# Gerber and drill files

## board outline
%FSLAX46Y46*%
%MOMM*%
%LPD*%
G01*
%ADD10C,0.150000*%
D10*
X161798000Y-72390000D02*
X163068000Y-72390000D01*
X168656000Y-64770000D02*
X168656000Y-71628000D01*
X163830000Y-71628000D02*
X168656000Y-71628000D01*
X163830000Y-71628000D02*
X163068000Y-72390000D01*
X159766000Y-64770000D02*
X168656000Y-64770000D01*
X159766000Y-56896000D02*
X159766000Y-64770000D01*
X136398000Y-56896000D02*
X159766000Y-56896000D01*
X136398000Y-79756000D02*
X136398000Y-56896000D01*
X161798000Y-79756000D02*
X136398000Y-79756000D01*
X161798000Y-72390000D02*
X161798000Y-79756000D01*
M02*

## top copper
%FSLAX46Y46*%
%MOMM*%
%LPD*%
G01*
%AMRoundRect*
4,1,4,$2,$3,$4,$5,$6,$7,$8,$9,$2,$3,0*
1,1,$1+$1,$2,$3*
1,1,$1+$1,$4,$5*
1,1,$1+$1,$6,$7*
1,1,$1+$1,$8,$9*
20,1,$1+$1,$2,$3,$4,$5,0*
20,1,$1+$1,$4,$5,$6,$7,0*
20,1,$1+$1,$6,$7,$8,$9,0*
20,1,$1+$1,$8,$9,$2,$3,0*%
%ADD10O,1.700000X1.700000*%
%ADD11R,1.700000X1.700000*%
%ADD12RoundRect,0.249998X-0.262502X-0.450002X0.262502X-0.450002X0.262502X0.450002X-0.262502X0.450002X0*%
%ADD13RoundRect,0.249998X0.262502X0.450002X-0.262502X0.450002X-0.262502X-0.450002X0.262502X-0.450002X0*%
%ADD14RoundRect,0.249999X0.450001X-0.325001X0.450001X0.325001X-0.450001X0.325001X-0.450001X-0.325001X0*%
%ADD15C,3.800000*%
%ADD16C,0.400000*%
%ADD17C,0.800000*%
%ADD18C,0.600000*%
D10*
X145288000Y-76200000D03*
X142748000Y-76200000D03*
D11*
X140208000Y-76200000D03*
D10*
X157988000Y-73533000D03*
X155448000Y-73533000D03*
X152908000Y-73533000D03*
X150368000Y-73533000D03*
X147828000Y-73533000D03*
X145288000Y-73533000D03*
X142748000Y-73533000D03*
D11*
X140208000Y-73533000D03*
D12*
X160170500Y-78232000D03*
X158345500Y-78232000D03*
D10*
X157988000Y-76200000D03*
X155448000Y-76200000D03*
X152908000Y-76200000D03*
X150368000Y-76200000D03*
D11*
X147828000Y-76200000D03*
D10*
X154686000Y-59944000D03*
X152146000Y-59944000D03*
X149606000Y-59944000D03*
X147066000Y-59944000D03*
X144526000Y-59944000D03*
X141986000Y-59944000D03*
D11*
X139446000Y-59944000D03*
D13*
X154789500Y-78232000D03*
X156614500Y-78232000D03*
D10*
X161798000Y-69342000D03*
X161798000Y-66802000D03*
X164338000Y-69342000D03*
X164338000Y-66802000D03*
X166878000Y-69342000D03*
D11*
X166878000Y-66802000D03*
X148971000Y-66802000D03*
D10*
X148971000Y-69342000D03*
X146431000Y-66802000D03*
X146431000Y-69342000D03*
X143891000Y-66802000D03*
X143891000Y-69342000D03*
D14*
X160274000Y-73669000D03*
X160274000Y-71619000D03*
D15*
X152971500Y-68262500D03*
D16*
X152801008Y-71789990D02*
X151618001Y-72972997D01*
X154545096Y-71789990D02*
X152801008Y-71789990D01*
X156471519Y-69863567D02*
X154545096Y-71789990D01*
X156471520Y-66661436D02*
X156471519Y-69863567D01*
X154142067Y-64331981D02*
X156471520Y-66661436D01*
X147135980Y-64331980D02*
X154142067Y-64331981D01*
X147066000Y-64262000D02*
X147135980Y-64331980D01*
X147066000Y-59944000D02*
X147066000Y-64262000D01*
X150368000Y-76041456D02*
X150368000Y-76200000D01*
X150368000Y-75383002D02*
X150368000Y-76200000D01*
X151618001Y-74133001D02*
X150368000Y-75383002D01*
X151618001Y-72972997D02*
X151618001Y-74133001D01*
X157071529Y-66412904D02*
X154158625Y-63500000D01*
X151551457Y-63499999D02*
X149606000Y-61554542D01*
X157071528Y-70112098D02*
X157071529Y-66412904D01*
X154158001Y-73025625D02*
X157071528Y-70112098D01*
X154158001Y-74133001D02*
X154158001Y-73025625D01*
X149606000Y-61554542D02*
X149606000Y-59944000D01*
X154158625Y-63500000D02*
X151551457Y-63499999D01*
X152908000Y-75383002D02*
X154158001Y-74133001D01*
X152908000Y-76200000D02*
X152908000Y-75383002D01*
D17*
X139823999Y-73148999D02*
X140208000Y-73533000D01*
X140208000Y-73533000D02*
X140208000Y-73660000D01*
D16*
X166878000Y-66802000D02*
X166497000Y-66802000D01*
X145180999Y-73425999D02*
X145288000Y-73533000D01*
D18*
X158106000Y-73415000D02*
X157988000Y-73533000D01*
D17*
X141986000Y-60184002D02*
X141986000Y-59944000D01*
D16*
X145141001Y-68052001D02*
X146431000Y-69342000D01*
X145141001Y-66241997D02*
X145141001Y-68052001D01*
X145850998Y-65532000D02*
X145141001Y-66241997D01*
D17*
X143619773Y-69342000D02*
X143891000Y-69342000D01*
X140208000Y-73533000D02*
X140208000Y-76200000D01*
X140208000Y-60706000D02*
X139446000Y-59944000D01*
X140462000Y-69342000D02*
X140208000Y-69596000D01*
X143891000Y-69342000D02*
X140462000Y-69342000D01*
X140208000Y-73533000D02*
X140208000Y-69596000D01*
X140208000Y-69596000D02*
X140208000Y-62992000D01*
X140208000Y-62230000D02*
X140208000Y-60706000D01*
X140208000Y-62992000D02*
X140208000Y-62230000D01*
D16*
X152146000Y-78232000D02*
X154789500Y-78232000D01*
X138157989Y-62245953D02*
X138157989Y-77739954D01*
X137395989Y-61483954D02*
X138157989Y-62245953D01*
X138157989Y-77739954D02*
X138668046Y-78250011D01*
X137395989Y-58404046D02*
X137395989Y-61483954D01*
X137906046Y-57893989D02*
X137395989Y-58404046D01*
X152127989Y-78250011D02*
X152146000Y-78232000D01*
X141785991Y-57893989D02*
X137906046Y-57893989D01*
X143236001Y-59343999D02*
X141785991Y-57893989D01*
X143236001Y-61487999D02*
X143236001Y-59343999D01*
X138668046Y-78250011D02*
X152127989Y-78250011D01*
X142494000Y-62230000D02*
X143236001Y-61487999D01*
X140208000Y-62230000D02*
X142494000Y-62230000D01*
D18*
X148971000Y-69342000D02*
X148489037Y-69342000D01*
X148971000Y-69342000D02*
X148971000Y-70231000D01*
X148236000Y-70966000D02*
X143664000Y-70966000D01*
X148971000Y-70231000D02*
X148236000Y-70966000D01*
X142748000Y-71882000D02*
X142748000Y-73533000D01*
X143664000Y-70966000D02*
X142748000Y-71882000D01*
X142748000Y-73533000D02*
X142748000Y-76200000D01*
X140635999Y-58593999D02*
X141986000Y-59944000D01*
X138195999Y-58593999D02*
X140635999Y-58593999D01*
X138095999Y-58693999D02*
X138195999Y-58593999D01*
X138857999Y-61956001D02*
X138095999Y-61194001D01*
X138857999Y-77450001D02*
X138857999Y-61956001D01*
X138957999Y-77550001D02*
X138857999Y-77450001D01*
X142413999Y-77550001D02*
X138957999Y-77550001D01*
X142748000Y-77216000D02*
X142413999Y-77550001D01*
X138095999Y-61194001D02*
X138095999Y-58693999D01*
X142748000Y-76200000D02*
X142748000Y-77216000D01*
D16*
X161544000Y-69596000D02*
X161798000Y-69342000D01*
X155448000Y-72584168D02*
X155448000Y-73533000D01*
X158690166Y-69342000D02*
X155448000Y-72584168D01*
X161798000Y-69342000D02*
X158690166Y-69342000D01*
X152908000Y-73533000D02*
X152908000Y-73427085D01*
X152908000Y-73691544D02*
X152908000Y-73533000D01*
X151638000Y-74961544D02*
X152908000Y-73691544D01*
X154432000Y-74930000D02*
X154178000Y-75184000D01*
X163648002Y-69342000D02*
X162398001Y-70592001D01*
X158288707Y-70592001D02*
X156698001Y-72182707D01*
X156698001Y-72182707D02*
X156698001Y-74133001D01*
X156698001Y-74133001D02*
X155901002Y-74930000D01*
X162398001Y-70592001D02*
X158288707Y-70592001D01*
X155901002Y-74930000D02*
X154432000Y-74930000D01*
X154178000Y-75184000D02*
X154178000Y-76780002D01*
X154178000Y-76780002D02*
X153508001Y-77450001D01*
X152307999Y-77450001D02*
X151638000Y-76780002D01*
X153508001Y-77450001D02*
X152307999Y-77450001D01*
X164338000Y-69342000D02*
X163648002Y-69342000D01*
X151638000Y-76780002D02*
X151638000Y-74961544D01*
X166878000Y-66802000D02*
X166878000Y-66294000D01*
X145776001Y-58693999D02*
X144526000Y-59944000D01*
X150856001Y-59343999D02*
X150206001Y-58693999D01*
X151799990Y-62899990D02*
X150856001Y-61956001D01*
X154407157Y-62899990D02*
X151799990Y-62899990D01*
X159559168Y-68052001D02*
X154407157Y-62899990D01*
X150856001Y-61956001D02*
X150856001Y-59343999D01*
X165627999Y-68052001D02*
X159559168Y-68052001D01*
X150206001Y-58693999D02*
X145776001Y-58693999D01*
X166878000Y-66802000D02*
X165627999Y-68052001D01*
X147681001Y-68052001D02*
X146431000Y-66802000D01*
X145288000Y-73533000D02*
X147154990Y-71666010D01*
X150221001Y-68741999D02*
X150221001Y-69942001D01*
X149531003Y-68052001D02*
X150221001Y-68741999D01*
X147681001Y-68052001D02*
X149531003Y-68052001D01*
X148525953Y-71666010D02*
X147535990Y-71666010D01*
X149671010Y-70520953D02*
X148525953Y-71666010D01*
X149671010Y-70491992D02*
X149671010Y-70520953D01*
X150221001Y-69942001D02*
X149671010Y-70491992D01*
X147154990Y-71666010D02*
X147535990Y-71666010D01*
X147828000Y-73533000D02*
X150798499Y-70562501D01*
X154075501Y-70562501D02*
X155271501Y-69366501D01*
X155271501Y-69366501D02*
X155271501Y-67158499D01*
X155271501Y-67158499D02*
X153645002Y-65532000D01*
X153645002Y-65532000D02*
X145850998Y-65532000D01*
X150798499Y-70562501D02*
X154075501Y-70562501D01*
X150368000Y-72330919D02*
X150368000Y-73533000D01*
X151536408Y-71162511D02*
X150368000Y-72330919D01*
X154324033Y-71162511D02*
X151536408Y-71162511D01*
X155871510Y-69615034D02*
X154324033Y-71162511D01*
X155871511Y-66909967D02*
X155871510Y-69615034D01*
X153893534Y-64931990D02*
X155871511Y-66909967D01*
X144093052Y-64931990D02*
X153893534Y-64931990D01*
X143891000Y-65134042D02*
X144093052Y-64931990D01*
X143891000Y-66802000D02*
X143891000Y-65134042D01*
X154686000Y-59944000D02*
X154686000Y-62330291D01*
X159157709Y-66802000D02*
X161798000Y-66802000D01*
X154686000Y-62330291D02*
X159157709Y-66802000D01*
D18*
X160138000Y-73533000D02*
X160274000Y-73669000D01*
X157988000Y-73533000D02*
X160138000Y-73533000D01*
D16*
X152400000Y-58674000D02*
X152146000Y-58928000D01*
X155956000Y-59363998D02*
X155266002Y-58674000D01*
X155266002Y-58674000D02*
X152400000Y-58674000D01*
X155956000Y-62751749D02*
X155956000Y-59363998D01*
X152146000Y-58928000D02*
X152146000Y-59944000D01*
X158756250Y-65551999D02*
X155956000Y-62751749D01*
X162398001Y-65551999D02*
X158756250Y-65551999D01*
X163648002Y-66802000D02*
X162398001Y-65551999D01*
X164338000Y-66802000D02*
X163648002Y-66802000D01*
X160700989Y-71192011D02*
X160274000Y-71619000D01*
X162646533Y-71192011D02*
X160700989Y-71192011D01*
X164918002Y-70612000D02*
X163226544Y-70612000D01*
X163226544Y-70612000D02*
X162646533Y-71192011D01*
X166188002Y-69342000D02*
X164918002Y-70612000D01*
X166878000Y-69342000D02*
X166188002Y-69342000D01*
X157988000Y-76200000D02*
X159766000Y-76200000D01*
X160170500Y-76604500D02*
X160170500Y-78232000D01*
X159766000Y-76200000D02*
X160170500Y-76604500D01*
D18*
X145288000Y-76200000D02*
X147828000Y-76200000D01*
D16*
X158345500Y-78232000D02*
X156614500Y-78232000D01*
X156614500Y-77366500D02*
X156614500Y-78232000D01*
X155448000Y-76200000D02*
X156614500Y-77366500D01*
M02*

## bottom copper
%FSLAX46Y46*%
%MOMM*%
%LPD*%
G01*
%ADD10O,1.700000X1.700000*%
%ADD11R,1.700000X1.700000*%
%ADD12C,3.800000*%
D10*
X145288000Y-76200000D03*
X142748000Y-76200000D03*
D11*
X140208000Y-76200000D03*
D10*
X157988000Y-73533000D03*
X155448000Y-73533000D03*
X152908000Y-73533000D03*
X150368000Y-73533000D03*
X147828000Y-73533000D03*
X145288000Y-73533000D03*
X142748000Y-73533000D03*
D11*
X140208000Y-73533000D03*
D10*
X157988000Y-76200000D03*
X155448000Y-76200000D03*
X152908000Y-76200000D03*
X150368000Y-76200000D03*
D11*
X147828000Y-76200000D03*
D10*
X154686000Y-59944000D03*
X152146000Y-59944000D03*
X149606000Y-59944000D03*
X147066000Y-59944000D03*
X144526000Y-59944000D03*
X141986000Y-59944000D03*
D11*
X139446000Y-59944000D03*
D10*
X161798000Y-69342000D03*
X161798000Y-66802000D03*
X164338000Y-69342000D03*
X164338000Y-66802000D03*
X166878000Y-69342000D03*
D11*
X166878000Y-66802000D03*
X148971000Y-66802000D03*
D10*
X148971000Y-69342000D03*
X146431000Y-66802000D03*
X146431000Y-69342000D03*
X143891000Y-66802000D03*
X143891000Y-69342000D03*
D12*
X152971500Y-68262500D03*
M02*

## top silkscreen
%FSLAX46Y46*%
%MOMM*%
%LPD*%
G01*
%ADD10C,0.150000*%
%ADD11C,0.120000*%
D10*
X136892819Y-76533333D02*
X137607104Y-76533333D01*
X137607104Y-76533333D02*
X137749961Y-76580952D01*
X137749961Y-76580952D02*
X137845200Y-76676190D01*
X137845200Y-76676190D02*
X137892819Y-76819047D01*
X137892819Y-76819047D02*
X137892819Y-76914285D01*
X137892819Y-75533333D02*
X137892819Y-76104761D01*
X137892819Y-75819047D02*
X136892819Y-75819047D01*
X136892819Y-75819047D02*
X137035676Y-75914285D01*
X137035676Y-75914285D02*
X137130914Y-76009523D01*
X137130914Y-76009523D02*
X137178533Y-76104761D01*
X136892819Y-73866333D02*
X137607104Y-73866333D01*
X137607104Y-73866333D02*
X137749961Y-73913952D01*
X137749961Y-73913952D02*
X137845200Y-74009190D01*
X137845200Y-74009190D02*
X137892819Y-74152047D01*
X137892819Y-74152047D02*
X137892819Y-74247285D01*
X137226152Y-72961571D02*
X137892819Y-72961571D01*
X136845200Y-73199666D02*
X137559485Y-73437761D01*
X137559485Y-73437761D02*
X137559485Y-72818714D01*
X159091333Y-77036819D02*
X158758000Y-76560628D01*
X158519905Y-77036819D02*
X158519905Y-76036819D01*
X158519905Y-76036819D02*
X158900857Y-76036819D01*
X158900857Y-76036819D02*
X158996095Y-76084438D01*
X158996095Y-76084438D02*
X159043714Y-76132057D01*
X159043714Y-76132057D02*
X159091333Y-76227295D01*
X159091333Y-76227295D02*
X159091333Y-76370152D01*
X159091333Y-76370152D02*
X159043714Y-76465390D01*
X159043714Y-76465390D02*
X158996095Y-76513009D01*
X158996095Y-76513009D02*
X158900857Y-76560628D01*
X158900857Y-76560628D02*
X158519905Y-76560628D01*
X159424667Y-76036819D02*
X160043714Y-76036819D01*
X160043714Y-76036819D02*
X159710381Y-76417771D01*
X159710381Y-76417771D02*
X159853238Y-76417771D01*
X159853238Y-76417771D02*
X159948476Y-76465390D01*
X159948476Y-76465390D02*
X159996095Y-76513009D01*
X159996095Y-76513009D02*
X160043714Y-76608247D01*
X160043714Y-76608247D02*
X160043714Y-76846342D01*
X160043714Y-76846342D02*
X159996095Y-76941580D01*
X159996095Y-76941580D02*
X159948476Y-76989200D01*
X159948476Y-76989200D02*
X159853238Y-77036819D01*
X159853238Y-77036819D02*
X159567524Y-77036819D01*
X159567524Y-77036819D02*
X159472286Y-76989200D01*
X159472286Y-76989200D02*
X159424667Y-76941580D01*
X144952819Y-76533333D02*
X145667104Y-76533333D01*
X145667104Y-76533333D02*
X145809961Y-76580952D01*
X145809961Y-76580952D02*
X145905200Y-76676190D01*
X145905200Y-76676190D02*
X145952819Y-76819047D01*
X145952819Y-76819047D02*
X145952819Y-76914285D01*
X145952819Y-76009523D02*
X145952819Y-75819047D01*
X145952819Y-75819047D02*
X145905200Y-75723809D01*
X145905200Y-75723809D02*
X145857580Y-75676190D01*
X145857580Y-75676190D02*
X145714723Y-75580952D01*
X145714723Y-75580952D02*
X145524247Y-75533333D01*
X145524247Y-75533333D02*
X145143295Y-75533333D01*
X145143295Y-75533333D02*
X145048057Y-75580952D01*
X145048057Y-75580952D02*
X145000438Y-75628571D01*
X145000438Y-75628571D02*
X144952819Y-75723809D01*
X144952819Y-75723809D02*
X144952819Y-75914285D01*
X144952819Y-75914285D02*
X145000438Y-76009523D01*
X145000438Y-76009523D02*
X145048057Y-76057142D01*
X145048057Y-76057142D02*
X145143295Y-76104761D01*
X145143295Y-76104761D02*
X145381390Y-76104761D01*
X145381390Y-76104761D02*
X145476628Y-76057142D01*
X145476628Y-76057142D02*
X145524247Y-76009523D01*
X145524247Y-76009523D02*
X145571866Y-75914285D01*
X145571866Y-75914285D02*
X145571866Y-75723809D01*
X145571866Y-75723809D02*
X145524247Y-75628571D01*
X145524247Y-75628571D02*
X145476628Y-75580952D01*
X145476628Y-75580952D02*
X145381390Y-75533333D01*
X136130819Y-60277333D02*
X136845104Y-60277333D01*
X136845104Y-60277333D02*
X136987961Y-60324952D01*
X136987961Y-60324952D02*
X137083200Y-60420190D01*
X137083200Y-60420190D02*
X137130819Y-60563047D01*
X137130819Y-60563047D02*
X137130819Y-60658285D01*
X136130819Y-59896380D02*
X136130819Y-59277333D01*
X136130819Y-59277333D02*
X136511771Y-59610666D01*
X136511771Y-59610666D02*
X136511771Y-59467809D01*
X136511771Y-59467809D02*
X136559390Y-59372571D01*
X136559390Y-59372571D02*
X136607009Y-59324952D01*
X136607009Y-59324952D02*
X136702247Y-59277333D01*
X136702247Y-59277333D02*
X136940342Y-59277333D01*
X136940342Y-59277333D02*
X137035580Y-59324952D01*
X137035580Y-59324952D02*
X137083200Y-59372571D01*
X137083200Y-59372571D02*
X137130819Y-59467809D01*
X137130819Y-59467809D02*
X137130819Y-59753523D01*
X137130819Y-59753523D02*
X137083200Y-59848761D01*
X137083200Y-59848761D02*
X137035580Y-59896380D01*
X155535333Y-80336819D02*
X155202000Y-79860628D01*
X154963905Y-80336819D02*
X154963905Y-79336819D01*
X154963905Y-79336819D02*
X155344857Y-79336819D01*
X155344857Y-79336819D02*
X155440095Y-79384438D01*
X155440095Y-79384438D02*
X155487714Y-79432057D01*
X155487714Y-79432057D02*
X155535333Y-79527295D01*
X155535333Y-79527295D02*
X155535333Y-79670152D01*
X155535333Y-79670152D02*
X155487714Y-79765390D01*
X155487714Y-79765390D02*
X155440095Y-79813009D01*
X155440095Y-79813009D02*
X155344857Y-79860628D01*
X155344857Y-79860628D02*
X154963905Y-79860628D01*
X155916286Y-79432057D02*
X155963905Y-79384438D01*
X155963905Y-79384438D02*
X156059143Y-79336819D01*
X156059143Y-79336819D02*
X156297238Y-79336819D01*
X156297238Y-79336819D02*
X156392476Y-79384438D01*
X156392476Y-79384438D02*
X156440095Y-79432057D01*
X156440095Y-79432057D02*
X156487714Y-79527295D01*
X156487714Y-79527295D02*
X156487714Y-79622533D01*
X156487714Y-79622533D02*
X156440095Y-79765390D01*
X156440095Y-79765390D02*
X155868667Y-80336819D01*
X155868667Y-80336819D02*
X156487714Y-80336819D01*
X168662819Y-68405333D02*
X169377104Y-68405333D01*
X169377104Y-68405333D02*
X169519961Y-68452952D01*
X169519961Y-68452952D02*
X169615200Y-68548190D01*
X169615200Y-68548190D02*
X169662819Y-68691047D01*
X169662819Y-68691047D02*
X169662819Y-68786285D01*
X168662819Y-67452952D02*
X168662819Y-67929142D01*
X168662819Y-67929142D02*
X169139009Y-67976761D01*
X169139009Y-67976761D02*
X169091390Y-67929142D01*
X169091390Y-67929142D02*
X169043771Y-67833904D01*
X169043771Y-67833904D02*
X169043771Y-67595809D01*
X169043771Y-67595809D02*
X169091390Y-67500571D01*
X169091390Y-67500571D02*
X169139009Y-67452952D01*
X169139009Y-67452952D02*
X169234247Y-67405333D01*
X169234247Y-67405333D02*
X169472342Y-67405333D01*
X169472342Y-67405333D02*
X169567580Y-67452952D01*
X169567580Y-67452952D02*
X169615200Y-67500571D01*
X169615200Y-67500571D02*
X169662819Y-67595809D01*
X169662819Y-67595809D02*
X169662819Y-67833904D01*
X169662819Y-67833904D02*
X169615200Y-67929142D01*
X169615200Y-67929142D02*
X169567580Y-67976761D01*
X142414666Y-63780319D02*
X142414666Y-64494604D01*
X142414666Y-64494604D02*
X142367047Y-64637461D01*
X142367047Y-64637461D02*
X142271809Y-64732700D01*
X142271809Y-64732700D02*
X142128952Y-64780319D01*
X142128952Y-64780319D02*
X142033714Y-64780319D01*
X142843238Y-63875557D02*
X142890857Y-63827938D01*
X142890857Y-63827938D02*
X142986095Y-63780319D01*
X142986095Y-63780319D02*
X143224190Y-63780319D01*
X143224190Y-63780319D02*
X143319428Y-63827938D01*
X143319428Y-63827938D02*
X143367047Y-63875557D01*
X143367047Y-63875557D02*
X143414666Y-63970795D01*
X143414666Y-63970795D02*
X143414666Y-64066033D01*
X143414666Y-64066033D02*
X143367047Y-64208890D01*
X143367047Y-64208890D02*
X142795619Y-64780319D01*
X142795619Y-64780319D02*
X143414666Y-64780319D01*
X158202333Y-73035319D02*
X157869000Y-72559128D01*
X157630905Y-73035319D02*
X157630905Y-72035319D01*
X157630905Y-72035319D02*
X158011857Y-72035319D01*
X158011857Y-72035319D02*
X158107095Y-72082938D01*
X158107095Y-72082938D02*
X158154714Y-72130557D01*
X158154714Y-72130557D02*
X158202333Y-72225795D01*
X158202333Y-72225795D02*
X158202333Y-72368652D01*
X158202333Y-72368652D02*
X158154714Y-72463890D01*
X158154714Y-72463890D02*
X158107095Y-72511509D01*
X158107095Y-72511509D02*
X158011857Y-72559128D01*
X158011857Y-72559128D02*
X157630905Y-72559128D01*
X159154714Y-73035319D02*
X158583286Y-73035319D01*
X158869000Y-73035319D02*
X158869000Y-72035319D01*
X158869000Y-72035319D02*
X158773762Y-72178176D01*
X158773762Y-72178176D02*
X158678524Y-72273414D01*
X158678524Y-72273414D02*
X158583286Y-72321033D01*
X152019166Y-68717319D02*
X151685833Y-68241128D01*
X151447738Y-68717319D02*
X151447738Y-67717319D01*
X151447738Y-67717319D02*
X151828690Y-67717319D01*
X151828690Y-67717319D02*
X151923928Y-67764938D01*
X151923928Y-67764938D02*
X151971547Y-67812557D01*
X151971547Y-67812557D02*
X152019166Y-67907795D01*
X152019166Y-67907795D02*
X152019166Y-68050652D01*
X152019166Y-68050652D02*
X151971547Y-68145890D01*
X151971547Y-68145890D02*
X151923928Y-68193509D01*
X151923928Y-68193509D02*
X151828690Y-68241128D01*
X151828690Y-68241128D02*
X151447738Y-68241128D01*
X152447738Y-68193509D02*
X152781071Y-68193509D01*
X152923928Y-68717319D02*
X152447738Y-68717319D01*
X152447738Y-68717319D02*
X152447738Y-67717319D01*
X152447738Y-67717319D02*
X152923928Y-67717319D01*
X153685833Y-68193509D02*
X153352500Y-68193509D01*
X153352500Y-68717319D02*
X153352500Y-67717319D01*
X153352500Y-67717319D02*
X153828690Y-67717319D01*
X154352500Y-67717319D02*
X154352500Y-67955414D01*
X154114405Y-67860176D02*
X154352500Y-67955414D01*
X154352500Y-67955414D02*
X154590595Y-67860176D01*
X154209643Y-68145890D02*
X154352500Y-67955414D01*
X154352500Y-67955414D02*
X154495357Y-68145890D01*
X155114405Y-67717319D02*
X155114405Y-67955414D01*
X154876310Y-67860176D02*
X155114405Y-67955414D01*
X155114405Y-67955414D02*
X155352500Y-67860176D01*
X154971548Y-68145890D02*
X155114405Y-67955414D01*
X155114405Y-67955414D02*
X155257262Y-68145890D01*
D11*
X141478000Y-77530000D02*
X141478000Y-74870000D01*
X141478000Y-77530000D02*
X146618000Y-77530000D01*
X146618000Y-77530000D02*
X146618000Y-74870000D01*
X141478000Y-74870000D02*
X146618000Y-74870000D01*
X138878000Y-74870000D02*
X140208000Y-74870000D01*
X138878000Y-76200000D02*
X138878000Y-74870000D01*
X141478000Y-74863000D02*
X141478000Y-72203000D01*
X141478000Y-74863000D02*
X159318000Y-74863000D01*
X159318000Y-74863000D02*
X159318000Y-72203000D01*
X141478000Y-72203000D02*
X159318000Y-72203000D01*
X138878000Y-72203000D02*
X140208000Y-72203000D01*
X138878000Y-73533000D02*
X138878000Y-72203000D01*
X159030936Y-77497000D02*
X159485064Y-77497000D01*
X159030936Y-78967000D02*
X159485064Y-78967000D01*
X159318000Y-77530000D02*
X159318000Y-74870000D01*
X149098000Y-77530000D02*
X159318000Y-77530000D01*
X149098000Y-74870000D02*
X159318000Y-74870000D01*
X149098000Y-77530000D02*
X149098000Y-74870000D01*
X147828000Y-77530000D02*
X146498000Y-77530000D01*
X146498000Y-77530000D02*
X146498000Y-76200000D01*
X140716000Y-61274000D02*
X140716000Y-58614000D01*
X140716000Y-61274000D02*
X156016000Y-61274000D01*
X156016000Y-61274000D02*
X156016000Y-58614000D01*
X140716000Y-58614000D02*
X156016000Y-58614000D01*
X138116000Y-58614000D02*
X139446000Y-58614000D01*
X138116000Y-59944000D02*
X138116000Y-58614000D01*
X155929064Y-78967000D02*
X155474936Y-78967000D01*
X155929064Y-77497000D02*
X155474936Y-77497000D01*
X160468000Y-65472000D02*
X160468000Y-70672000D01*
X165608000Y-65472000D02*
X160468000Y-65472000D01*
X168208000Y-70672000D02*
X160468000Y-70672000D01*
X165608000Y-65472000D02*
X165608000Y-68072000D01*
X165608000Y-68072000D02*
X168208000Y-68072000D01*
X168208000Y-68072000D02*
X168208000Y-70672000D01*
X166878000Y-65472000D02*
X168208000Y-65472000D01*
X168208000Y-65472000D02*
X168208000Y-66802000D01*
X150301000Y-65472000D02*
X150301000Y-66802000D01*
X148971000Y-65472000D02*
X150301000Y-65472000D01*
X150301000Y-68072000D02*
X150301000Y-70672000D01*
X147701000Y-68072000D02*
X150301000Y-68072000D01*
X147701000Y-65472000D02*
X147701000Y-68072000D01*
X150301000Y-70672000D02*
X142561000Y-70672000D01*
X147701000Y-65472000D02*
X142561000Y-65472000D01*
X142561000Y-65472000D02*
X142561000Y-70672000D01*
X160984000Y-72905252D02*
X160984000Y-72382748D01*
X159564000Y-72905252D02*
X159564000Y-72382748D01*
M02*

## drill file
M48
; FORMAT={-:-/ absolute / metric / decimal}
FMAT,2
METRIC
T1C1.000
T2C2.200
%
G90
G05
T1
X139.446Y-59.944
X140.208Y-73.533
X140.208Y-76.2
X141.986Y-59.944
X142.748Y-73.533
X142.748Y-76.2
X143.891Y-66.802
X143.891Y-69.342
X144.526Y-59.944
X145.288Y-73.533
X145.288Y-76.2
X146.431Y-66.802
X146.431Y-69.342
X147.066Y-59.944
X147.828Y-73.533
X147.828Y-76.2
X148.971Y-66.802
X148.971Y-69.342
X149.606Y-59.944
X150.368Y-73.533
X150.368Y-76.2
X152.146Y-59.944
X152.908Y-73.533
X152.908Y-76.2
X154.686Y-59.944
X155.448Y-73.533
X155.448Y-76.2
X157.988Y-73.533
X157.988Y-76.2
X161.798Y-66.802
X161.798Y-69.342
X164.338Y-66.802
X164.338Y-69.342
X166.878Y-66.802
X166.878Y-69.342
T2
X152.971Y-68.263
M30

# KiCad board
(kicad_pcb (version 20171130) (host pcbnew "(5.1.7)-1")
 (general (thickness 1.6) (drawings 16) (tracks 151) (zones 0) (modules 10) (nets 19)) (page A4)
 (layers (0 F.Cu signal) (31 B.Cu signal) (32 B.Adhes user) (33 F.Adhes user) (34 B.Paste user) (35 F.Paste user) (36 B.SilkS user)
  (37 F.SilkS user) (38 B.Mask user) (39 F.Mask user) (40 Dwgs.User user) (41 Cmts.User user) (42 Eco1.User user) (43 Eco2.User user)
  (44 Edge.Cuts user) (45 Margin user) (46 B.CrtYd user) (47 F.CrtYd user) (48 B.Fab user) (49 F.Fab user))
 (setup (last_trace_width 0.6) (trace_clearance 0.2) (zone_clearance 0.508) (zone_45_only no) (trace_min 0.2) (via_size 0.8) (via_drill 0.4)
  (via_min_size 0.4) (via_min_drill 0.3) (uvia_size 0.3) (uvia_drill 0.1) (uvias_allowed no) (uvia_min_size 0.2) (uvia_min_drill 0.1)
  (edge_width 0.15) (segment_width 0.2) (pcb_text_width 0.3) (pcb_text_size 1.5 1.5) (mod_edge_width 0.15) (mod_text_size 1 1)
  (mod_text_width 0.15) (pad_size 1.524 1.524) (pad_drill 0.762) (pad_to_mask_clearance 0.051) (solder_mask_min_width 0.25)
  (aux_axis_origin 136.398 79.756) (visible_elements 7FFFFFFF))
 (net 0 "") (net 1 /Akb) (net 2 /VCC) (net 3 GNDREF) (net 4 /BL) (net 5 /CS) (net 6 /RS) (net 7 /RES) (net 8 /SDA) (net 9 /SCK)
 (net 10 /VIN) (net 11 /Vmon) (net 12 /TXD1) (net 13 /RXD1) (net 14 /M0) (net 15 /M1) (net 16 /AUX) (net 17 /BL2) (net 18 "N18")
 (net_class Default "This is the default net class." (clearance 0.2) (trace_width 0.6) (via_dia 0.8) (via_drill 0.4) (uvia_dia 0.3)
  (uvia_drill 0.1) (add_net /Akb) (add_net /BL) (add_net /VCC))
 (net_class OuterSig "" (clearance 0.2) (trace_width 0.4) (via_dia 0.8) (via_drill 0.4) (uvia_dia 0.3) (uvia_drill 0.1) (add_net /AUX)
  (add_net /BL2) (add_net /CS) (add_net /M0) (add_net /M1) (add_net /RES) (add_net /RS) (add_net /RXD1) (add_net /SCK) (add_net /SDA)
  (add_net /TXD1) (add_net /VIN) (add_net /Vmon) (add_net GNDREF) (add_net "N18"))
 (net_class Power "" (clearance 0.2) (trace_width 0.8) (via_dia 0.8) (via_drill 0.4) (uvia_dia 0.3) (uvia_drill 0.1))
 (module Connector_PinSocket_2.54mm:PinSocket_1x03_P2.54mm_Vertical (layer F.Cu) (at 140.208 76.2 90)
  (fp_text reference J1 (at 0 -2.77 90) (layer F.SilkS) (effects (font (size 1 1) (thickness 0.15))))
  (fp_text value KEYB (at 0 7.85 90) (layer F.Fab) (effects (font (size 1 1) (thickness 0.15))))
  (fp_line (start -1.33 1.27) (end 1.33 1.27) (layer F.SilkS) (width 0.12))
  (fp_line (start -1.33 1.27) (end -1.33 6.41) (layer F.SilkS) (width 0.12))
  (fp_line (start -1.33 6.41) (end 1.33 6.41) (layer F.SilkS) (width 0.12))
  (fp_line (start 1.33 1.27) (end 1.33 6.41) (layer F.SilkS) (width 0.12))
  (fp_line (start 1.33 -1.33) (end 1.33 0) (layer F.SilkS) (width 0.12))
  (fp_line (start 0 -1.33) (end 1.33 -1.33) (layer F.SilkS) (width 0.12))
  (pad 3 thru_hole oval (at 0 5.08 90) (size 1.7 1.7) (drill 1) (layers *.Cu *.Mask) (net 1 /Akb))
  (pad 2 thru_hole oval (at 0 2.54 90) (size 1.7 1.7) (drill 1) (layers *.Cu *.Mask) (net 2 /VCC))
  (pad 1 thru_hole rect (at 0 0 90) (size 1.7 1.7) (drill 1) (layers *.Cu *.Mask) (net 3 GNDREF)))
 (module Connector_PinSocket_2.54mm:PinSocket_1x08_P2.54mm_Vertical (layer F.Cu) (at 140.208 73.533 90)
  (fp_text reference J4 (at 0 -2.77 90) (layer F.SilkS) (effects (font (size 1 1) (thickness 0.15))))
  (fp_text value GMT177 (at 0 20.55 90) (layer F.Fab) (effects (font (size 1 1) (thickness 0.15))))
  (fp_line (start -1.33 1.27) (end 1.33 1.27) (layer F.SilkS) (width 0.12))
  (fp_line (start -1.33 1.27) (end -1.33 19.11) (layer F.SilkS) (width 0.12))
  (fp_line (start -1.33 19.11) (end 1.33 19.11) (layer F.SilkS) (width 0.12))
  (fp_line (start 1.33 1.27) (end 1.33 19.11) (layer F.SilkS) (width 0.12))
  (fp_line (start 1.33 -1.33) (end 1.33 0) (layer F.SilkS) (width 0.12))
  (fp_line (start 0 -1.33) (end 1.33 -1.33) (layer F.SilkS) (width 0.12))
  (pad 8 thru_hole oval (at 0 17.78 90) (size 1.7 1.7) (drill 1) (layers *.Cu *.Mask) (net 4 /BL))
  (pad 7 thru_hole oval (at 0 15.24 90) (size 1.7 1.7) (drill 1) (layers *.Cu *.Mask) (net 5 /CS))
  (pad 6 thru_hole oval (at 0 12.7 90) (size 1.7 1.7) (drill 1) (layers *.Cu *.Mask) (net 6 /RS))
  (pad 5 thru_hole oval (at 0 10.16 90) (size 1.7 1.7) (drill 1) (layers *.Cu *.Mask) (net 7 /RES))
  (pad 4 thru_hole oval (at 0 7.62 90) (size 1.7 1.7) (drill 1) (layers *.Cu *.Mask) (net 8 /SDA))
  (pad 3 thru_hole oval (at 0 5.08 90) (size 1.7 1.7) (drill 1) (layers *.Cu *.Mask) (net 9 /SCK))
  (pad 2 thru_hole oval (at 0 2.54 90) (size 1.7 1.7) (drill 1) (layers *.Cu *.Mask) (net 2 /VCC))
  (pad 1 thru_hole rect (at 0 0 90) (size 1.7 1.7) (drill 1) (layers *.Cu *.Mask) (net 3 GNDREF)))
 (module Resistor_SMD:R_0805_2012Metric (layer F.Cu) (at 159.258 78.232)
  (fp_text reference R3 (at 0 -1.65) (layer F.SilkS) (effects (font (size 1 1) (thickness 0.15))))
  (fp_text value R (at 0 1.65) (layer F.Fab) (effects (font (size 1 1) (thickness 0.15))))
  (fp_line (start -0.227064 -0.735) (end 0.227064 -0.735) (layer F.SilkS) (width 0.12))
  (fp_line (start -0.227064 0.735) (end 0.227064 0.735) (layer F.SilkS) (width 0.12))
  (pad 2 smd roundrect (at 0.9125 0) (size 1.025 1.4) (layers F.Cu F.Paste F.Mask) (roundrect_rratio 0.2439004878048781) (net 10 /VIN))
  (pad 1 smd roundrect (at -0.9125 0) (size 1.025 1.4) (layers F.Cu F.Paste F.Mask) (roundrect_rratio 0.2439004878048781) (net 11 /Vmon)))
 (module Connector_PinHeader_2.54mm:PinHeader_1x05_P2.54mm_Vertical (layer F.Cu) (at 147.828 76.2 90)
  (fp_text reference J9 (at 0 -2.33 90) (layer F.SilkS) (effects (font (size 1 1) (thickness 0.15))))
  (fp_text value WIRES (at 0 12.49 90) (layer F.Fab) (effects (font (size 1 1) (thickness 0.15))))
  (fp_line (start -1.33 11.49) (end 1.33 11.49) (layer F.SilkS) (width 0.12))
  (fp_line (start -1.33 1.27) (end -1.33 11.49) (layer F.SilkS) (width 0.12))
  (fp_line (start 1.33 1.27) (end 1.33 11.49) (layer F.SilkS) (width 0.12))
  (fp_line (start -1.33 1.27) (end 1.33 1.27) (layer F.SilkS) (width 0.12))
  (fp_line (start -1.33 0) (end -1.33 -1.33) (layer F.SilkS) (width 0.12))
  (fp_line (start -1.33 -1.33) (end 0 -1.33) (layer F.SilkS) (width 0.12))
  (pad 5 thru_hole oval (at 0 10.16 90) (size 1.7 1.7) (drill 1) (layers *.Cu *.Mask) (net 10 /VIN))
  (pad 4 thru_hole oval (at 0 7.62 90) (size 1.7 1.7) (drill 1) (layers *.Cu *.Mask) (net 11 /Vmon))
  (pad 3 thru_hole oval (at 0 5.08 90) (size 1.7 1.7) (drill 1) (layers *.Cu *.Mask) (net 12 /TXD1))
  (pad 2 thru_hole oval (at 0 2.54 90) (size 1.7 1.7) (drill 1) (layers *.Cu *.Mask) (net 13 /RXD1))
  (pad 1 thru_hole rect (at 0 0 90) (size 1.7 1.7) (drill 1) (layers *.Cu *.Mask) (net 1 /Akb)))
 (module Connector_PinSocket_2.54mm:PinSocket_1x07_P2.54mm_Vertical (layer F.Cu) (at 139.446 59.944 90)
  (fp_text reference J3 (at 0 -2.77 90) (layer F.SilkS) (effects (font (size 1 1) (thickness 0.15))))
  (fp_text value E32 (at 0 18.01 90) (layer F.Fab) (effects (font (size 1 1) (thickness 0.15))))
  (fp_line (start -1.33 1.27) (end 1.33 1.27) (layer F.SilkS) (width 0.12))
  (fp_line (start -1.33 1.27) (end -1.33 16.57) (layer F.SilkS) (width 0.12))
  (fp_line (start -1.33 16.57) (end 1.33 16.57) (layer F.SilkS) (width 0.12))
  (fp_line (start 1.33 1.27) (end 1.33 16.57) (layer F.SilkS) (width 0.12))
  (fp_line (start 1.33 -1.33) (end 1.33 0) (layer F.SilkS) (width 0.12))
  (fp_line (start 0 -1.33) (end 1.33 -1.33) (layer F.SilkS) (width 0.12))
  (pad 7 thru_hole oval (at 0 15.24 90) (size 1.7 1.7) (drill 1) (layers *.Cu *.Mask) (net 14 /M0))
  (pad 6 thru_hole oval (at 0 12.7 90) (size 1.7 1.7) (drill 1) (layers *.Cu *.Mask) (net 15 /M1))
  (pad 5 thru_hole oval (at 0 10.16 90) (size 1.7 1.7) (drill 1) (layers *.Cu *.Mask) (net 12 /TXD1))
  (pad 4 thru_hole oval (at 0 7.62 90) (size 1.7 1.7) (drill 1) (layers *.Cu *.Mask) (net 13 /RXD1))
  (pad 3 thru_hole oval (at 0 5.08 90) (size 1.7 1.7) (drill 1) (layers *.Cu *.Mask) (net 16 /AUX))
  (pad 2 thru_hole oval (at 0 2.54 90) (size 1.7 1.7) (drill 1) (layers *.Cu *.Mask) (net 2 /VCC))
  (pad 1 thru_hole rect (at 0 0 90) (size 1.7 1.7) (drill 1) (layers *.Cu *.Mask) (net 3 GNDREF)))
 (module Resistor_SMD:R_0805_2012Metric (layer F.Cu) (at 155.702 78.232 180)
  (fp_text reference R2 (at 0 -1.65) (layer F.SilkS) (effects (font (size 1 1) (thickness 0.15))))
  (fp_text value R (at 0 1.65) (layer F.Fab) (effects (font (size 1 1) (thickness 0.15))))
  (fp_line (start -0.227064 -0.735) (end 0.227064 -0.735) (layer F.SilkS) (width 0.12))
  (fp_line (start -0.227064 0.735) (end 0.227064 0.735) (layer F.SilkS) (width 0.12))
  (pad 2 smd roundrect (at 0.9125 0 180) (size 1.025 1.4) (layers F.Cu F.Paste F.Mask) (roundrect_rratio 0.2439004878048781) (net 3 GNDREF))
  (pad 1 smd roundrect (at -0.9125 0 180) (size 1.025 1.4) (layers F.Cu F.Paste F.Mask) (roundrect_rratio 0.2439004878048781) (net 11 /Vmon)))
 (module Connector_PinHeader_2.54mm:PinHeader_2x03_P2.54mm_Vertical (layer F.Cu) (at 166.878 66.802 270)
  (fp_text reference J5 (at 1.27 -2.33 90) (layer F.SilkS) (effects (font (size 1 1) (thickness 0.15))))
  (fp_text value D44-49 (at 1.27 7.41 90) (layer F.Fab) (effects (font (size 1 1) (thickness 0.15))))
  (fp_line (start -1.33 6.41) (end 3.87 6.41) (layer F.SilkS) (width 0.12))
  (fp_line (start -1.33 1.27) (end -1.33 6.41) (layer F.SilkS) (width 0.12))
  (fp_line (start 3.87 -1.33) (end 3.87 6.41) (layer F.SilkS) (width 0.12))
  (fp_line (start -1.33 1.27) (end 1.27 1.27) (layer F.SilkS) (width 0.12))
  (fp_line (start 1.27 1.27) (end 1.27 -1.33) (layer F.SilkS) (width 0.12))
  (fp_line (start 1.27 -1.33) (end 3.87 -1.33) (layer F.SilkS) (width 0.12))
  (fp_line (start -1.33 0) (end -1.33 -1.33) (layer F.SilkS) (width 0.12))
  (fp_line (start -1.33 -1.33) (end 0 -1.33) (layer F.SilkS) (width 0.12))
  (pad 6 thru_hole oval (at 2.54 5.08 270) (size 1.7 1.7) (drill 1) (layers *.Cu *.Mask) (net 5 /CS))
  (pad 5 thru_hole oval (at 0 5.08 270) (size 1.7 1.7) (drill 1) (layers *.Cu *.Mask) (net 14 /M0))
  (pad 4 thru_hole oval (at 2.54 2.54 270) (size 1.7 1.7) (drill 1) (layers *.Cu *.Mask) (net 6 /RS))
  (pad 3 thru_hole oval (at 0 2.54 270) (size 1.7 1.7) (drill 1) (layers *.Cu *.Mask) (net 15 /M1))
  (pad 2 thru_hole oval (at 2.54 0 270) (size 1.7 1.7) (drill 1) (layers *.Cu *.Mask) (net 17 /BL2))
  (pad 1 thru_hole rect (at 0 0 270) (size 1.7 1.7) (drill 1) (layers *.Cu *.Mask) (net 16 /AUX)))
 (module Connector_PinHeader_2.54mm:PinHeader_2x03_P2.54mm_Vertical (layer F.Cu) (at 148.971 66.802 270)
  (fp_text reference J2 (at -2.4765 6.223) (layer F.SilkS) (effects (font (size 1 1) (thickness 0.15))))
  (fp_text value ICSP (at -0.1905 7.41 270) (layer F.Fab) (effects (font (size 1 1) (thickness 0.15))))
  (fp_line (start -1.33 -1.33) (end 0 -1.33) (layer F.SilkS) (width 0.12))
  (fp_line (start -1.33 0) (end -1.33 -1.33) (layer F.SilkS) (width 0.12))
  (fp_line (start 1.27 -1.33) (end 3.87 -1.33) (layer F.SilkS) (width 0.12))
  (fp_line (start 1.27 1.27) (end 1.27 -1.33) (layer F.SilkS) (width 0.12))
  (fp_line (start -1.33 1.27) (end 1.27 1.27) (layer F.SilkS) (width 0.12))
  (fp_line (start 3.87 -1.33) (end 3.87 6.41) (layer F.SilkS) (width 0.12))
  (fp_line (start -1.33 1.27) (end -1.33 6.41) (layer F.SilkS) (width 0.12))
  (fp_line (start -1.33 6.41) (end 3.87 6.41) (layer F.SilkS) (width 0.12))
  (pad 1 thru_hole rect (at 0 0 270) (size 1.7 1.7) (drill 1) (layers *.Cu *.Mask) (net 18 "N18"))
  (pad 2 thru_hole oval (at 2.54 0 270) (size 1.7 1.7) (drill 1) (layers *.Cu *.Mask) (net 2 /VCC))
  (pad 3 thru_hole oval (at 0 2.54 270) (size 1.7 1.7) (drill 1) (layers *.Cu *.Mask) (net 9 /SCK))
  (pad 4 thru_hole oval (at 2.54 2.54 270) (size 1.7 1.7) (drill 1) (layers *.Cu *.Mask) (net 8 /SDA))
  (pad 5 thru_hole oval (at 0 5.08 270) (size 1.7 1.7) (drill 1) (layers *.Cu *.Mask) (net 7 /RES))
  (pad 6 thru_hole oval (at 2.54 5.08 270) (size 1.7 1.7) (drill 1) (layers *.Cu *.Mask) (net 3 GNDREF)))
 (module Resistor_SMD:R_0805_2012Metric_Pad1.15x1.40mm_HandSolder (layer F.Cu) (at 160.274 72.644 90)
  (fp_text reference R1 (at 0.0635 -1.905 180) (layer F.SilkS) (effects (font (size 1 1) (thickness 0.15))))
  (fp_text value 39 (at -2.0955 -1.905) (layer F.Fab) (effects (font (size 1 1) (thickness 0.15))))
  (fp_line (start -0.261252 0.71) (end 0.261252 0.71) (layer F.SilkS) (width 0.12))
  (fp_line (start -0.261252 -0.71) (end 0.261252 -0.71) (layer F.SilkS) (width 0.12))
  (pad 1 smd roundrect (at -1.025 0 90) (size 1.15 1.4) (layers F.Cu F.Paste F.Mask) (roundrect_rratio 0.2173904347826087) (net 4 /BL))
  (pad 2 smd roundrect (at 1.025 0 90) (size 1.15 1.4) (layers F.Cu F.Paste F.Mask) (roundrect_rratio 0.2173904347826087) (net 17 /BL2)))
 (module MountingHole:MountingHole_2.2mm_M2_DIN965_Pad (layer F.Cu) (at 152.9715 68.2625)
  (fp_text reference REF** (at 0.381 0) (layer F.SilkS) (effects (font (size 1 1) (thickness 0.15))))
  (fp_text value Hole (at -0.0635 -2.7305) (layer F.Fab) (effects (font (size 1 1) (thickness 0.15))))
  (pad 1 thru_hole circle (at 0 0) (size 3.8 3.8) (drill 2.2) (layers *.Cu *.Mask)))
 (gr_line (start 161.798 72.39) (end 163.068 72.39) (layer Edge.Cuts) (width 0.15))
 (gr_line (start 168.656 64.77) (end 168.656 71.628) (layer Edge.Cuts) (width 0.15))
 (gr_line (start 163.83 71.628) (end 168.656 71.628) (layer Edge.Cuts) (width 0.15))
 (gr_line (start 163.83 71.628) (end 163.068 72.39) (layer Edge.Cuts) (width 0.15))
 (gr_line (start 159.766 64.77) (end 168.656 64.77) (layer Edge.Cuts) (width 0.15))
 (gr_line (start 159.766 56.896) (end 159.766 64.77) (layer Edge.Cuts) (width 0.15))
 (gr_line (start 136.398 56.896) (end 159.766 56.896) (layer Edge.Cuts) (width 0.15))
 (gr_line (start 136.398 79.756) (end 136.398 56.896) (layer Edge.Cuts) (width 0.15))
 (gr_line (start 161.798 79.756) (end 136.398 79.756) (layer Edge.Cuts) (width 0.15))
 (gr_line (start 161.798 72.39) (end 161.798 79.756) (layer Edge.Cuts) (width 0.15))
 (segment (start 152.801008 71.78999) (end 151.618001 72.972997) (width 0.4) (layer F.Cu) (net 13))
 (segment (start 154.545096 71.78999) (end 152.801008 71.78999) (width 0.4) (layer F.Cu) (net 13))
 (segment (start 156.471519 69.863567) (end 154.545096 71.78999) (width 0.4) (layer F.Cu) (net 13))
 (segment (start 156.47152 66.661436) (end 156.471519 69.863567) (width 0.4) (layer F.Cu) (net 13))
 (segment (start 154.142067 64.331981) (end 156.47152 66.661436) (width 0.4) (layer F.Cu) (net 13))
 (segment (start 147.13598 64.33198) (end 154.142067 64.331981) (width 0.4) (layer F.Cu) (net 13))
 (segment (start 147.066 64.262) (end 147.13598 64.33198) (width 0.4) (layer F.Cu) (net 13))
 (segment (start 147.066 59.944) (end 147.066 64.262) (width 0.4) (layer F.Cu) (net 13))
 (segment (start 150.368 76.041456) (end 150.368 76.2) (width 0.4) (layer F.Cu) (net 13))
 (segment (start 150.368 75.383002) (end 150.368 76.2) (width 0.4) (layer F.Cu) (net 13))
 (segment (start 151.618001 74.133001) (end 150.368 75.383002) (width 0.4) (layer F.Cu) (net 13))
 (segment (start 151.618001 72.972997) (end 151.618001 74.133001) (width 0.4) (layer F.Cu) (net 13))
 (segment (start 157.071529 66.412904) (end 154.158625 63.5) (width 0.4) (layer F.Cu) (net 12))
 (segment (start 151.551457 63.499999) (end 149.606 61.554542) (width 0.4) (layer F.Cu) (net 12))
 (segment (start 157.071528 70.112098) (end 157.071529 66.412904) (width 0.4) (layer F.Cu) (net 12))
 (segment (start 154.158001 73.025625) (end 157.071528 70.112098) (width 0.4) (layer F.Cu) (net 12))
 (segment (start 154.158001 74.133001) (end 154.158001 73.025625) (width 0.4) (layer F.Cu) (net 12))
 (segment (start 149.606 61.554542) (end 149.606 59.944) (width 0.4) (layer F.Cu) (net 12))
 (segment (start 154.158625 63.5) (end 151.551457 63.499999) (width 0.4) (layer F.Cu) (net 12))
 (segment (start 152.908 75.383002) (end 154.158001 74.133001) (width 0.4) (layer F.Cu) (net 12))
 (segment (start 152.908 76.2) (end 152.908 75.383002) (width 0.4) (layer F.Cu) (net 12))
 (segment (start 139.823999 73.148999) (end 140.208 73.533) (width 0.8) (layer F.Cu) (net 3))
 (segment (start 140.208 73.533) (end 140.208 73.66) (width 0.8) (layer F.Cu) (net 3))
 (segment (start 166.878 66.802) (end 166.497 66.802) (width 0.4) (layer F.Cu) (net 16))
 (segment (start 145.180999 73.425999) (end 145.288 73.533) (width 0.4) (layer F.Cu) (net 9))
 (segment (start 158.106 73.415) (end 157.988 73.533) (width 0.6) (layer F.Cu) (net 4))
 (segment (start 141.986 60.184002) (end 141.986 59.944) (width 0.8) (layer F.Cu) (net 2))
 (segment (start 145.141001 68.052001) (end 146.431 69.342) (width 0.4) (layer F.Cu) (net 8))
 (segment (start 145.141001 66.241997) (end 145.141001 68.052001) (width 0.4) (layer F.Cu) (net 8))
 (segment (start 145.850998 65.532) (end 145.141001 66.241997) (width 0.4) (layer F.Cu) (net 8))
 (segment (start 143.619773 69.342) (end 143.891 69.342) (width 0.8) (layer F.Cu) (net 3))
 (segment (start 140.208 73.533) (end 140.208 76.2) (width 0.8) (layer F.Cu) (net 3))
 (segment (start 140.208 60.706) (end 139.446 59.944) (width 0.8) (layer F.Cu) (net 3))
 (segment (start 140.462 69.342) (end 140.208 69.596) (width 0.8) (layer F.Cu) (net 3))
 (segment (start 143.891 69.342) (end 140.462 69.342) (width 0.8) (layer F.Cu) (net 3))
 (segment (start 140.208 73.533) (end 140.208 69.596) (width 0.8) (layer F.Cu) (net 3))
 (segment (start 140.208 69.596) (end 140.208 62.992) (width 0.8) (layer F.Cu) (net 3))
 (segment (start 140.208 62.23) (end 140.208 60.706) (width 0.8) (layer F.Cu) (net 3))
 (segment (start 140.208 62.992) (end 140.208 62.23) (width 0.8) (layer F.Cu) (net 3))
 (segment (start 152.146 78.232) (end 154.7895 78.232) (width 0.4) (layer F.Cu) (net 3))
 (segment (start 138.157989 62.245953) (end 138.157989 77.739954) (width 0.4) (layer F.Cu) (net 3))
 (segment (start 137.395989 61.483954) (end 138.157989 62.245953) (width 0.4) (layer F.Cu) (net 3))
 (segment (start 138.157989 77.739954) (end 138.668046 78.250011) (width 0.4) (layer F.Cu) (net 3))
 (segment (start 137.395989 58.404046) (end 137.395989 61.483954) (width 0.4) (layer F.Cu) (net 3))
 (segment (start 137.906046 57.893989) (end 137.395989 58.404046) (width 0.4) (layer F.Cu) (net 3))
 (segment (start 152.127989 78.250011) (end 152.146 78.232) (width 0.4) (layer F.Cu) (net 3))
 (segment (start 141.785991 57.893989) (end 137.906046 57.893989) (width 0.4) (layer F.Cu) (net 3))
 (segment (start 143.236001 59.343999) (end 141.785991 57.893989) (width 0.4) (layer F.Cu) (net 3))
 (segment (start 143.236001 61.487999) (end 143.236001 59.343999) (width 0.4) (layer F.Cu) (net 3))
 (segment (start 138.668046 78.250011) (end 152.127989 78.250011) (width 0.4) (layer F.Cu) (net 3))
 (segment (start 142.494 62.23) (end 143.236001 61.487999) (width 0.4) (layer F.Cu) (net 3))
 (segment (start 140.208 62.23) (end 142.494 62.23) (width 0.4) (layer F.Cu) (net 3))
 (segment (start 148.971 69.342) (end 148.489037 69.342) (width 0.6) (layer F.Cu) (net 2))
 (segment (start 148.971 69.342) (end 148.971 70.231) (width 0.6) (layer F.Cu) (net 2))
 (segment (start 148.236 70.966) (end 143.664 70.966) (width 0.6) (layer F.Cu) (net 2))
 (segment (start 148.971 70.231) (end 148.236 70.966) (width 0.6) (layer F.Cu) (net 2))
 (segment (start 142.748 71.882) (end 142.748 73.533) (width 0.6) (layer F.Cu) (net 2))
 (segment (start 143.664 70.966) (end 142.748 71.882) (width 0.6) (layer F.Cu) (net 2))
 (segment (start 142.748 73.533) (end 142.748 76.2) (width 0.6) (layer F.Cu) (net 2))
 (segment (start 140.635999 58.593999) (end 141.986 59.944) (width 0.6) (layer F.Cu) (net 2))
 (segment (start 138.195999 58.593999) (end 140.635999 58.593999) (width 0.6) (layer F.Cu) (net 2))
 (segment (start 138.095999 58.693999) (end 138.195999 58.593999) (width 0.6) (layer F.Cu) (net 2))
 (segment (start 138.857999 61.956001) (end 138.095999 61.194001) (width 0.6) (layer F.Cu) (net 2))
 (segment (start 138.857999 77.450001) (end 138.857999 61.956001) (width 0.6) (layer F.Cu) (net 2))
 (segment (start 138.957999 77.550001) (end 138.857999 77.450001) (width 0.6) (layer F.Cu) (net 2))
 (segment (start 142.413999 77.550001) (end 138.957999 77.550001) (width 0.6) (layer F.Cu) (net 2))
 (segment (start 142.748 77.216) (end 142.413999 77.550001) (width 0.6) (layer F.Cu) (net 2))
 (segment (start 138.095999 61.194001) (end 138.095999 58.693999) (width 0.6) (layer F.Cu) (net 2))
 (segment (start 142.748 76.2) (end 142.748 77.216) (width 0.6) (layer F.Cu) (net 2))
 (segment (start 161.544 69.596) (end 161.798 69.342) (width 0.4) (layer F.Cu) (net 5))
 (segment (start 155.448 72.584168) (end 155.448 73.533) (width 0.4) (layer F.Cu) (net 5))
 (segment (start 158.690166 69.342) (end 155.448 72.584168) (width 0.4) (layer F.Cu) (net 5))
 (segment (start 161.798 69.342) (end 158.690166 69.342) (width 0.4) (layer F.Cu) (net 5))
 (segment (start 152.908 73.533) (end 152.908 73.427085) (width 0.4) (layer F.Cu) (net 6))
 (segment (start 152.908 73.691544) (end 152.908 73.533) (width 0.4) (layer F.Cu) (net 6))
 (segment (start 151.638 74.961544) (end 152.908 73.691544) (width 0.4) (layer F.Cu) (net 6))
 (segment (start 154.432 74.93) (end 154.178 75.184) (width 0.4) (layer F.Cu) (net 6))
 (segment (start 163.648002 69.342) (end 162.398001 70.592001) (width 0.4) (layer F.Cu) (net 6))
 (segment (start 158.288707 70.592001) (end 156.698001 72.182707) (width 0.4) (layer F.Cu) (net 6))
 (segment (start 156.698001 72.182707) (end 156.698001 74.133001) (width 0.4) (layer F.Cu) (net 6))
 (segment (start 156.698001 74.133001) (end 155.901002 74.93) (width 0.4) (layer F.Cu) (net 6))
 (segment (start 162.398001 70.592001) (end 158.288707 70.592001) (width 0.4) (layer F.Cu) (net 6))
 (segment (start 155.901002 74.93) (end 154.432 74.93) (width 0.4) (layer F.Cu) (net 6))
 (segment (start 154.178 75.184) (end 154.178 76.780002) (width 0.4) (layer F.Cu) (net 6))
 (segment (start 154.178 76.780002) (end 153.508001 77.450001) (width 0.4) (layer F.Cu) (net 6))
 (segment (start 152.307999 77.450001) (end 151.638 76.780002) (width 0.4) (layer F.Cu) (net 6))
 (segment (start 153.508001 77.450001) (end 152.307999 77.450001) (width 0.4) (layer F.Cu) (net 6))
 (segment (start 164.338 69.342) (end 163.648002 69.342) (width 0.4) (layer F.Cu) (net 6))
 (segment (start 151.638 76.780002) (end 151.638 74.961544) (width 0.4) (layer F.Cu) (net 6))
 (segment (start 166.878 66.802) (end 166.878 66.294) (width 0.4) (layer F.Cu) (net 16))
 (segment (start 145.776001 58.693999) (end 144.526 59.944) (width 0.4) (layer F.Cu) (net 16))
 (segment (start 150.856001 59.343999) (end 150.206001 58.693999) (width 0.4) (layer F.Cu) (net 16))
 (segment (start 151.79999 62.89999) (end 150.856001 61.956001) (width 0.4) (layer F.Cu) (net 16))
 (segment (start 154.407157 62.89999) (end 151.79999 62.89999) (width 0.4) (layer F.Cu) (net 16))
 (segment (start 159.559168 68.052001) (end 154.407157 62.89999) (width 0.4) (layer F.Cu) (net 16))
 (segment (start 150.856001 61.956001) (end 150.856001 59.343999) (width 0.4) (layer F.Cu) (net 16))
 (segment (start 165.627999 68.052001) (end 159.559168 68.052001) (width 0.4) (layer F.Cu) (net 16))
 (segment (start 150.206001 58.693999) (end 145.776001 58.693999) (width 0.4) (layer F.Cu) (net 16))
 (segment (start 166.878 66.802) (end 165.627999 68.052001) (width 0.4) (layer F.Cu) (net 16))
 (segment (start 147.681001 68.052001) (end 146.431 66.802) (width 0.4) (layer F.Cu) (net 9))
 (segment (start 145.288 73.533) (end 147.15499 71.66601) (width 0.4) (layer F.Cu) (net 9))
 (segment (start 150.221001 68.741999) (end 150.221001 69.942001) (width 0.4) (layer F.Cu) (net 9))
 (segment (start 149.531003 68.052001) (end 150.221001 68.741999) (width 0.4) (layer F.Cu) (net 9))
 (segment (start 147.681001 68.052001) (end 149.531003 68.052001) (width 0.4) (layer F.Cu) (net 9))
 (segment (start 148.525953 71.66601) (end 147.53599 71.66601) (width 0.4) (layer F.Cu) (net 9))
 (segment (start 149.67101 70.520953) (end 148.525953 71.66601) (width 0.4) (layer F.Cu) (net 9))
 (segment (start 149.67101 70.491992) (end 149.67101 70.520953) (width 0.4) (layer F.Cu) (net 9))
 (segment (start 150.221001 69.942001) (end 149.67101 70.491992) (width 0.4) (layer F.Cu) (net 9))
 (segment (start 147.15499 71.66601) (end 147.53599 71.66601) (width 0.4) (layer F.Cu) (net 9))
 (segment (start 147.828 73.533) (end 150.798499 70.562501) (width 0.4) (layer F.Cu) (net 8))
 (segment (start 154.075501 70.562501) (end 155.271501 69.366501) (width 0.4) (layer F.Cu) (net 8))
 (segment (start 155.271501 69.366501) (end 155.271501 67.158499) (width 0.4) (layer F.Cu) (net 8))
 (segment (start 155.271501 67.158499) (end 153.645002 65.532) (width 0.4) (layer F.Cu) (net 8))
 (segment (start 153.645002 65.532) (end 145.850998 65.532) (width 0.4) (layer F.Cu) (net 8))
 (segment (start 150.798499 70.562501) (end 154.075501 70.562501) (width 0.4) (layer F.Cu) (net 8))
 (segment (start 150.368 72.330919) (end 150.368 73.533) (width 0.4) (layer F.Cu) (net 7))
 (segment (start 151.536408 71.162511) (end 150.368 72.330919) (width 0.4) (layer F.Cu) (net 7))
 (segment (start 154.324033 71.162511) (end 151.536408 71.162511) (width 0.4) (layer F.Cu) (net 7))
 (segment (start 155.87151 69.615034) (end 154.324033 71.162511) (width 0.4) (layer F.Cu) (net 7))
 (segment (start 155.871511 66.909967) (end 155.87151 69.615034) (width 0.4) (layer F.Cu) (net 7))
 (segment (start 153.893534 64.93199) (end 155.871511 66.909967) (width 0.4) (layer F.Cu) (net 7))
 (segment (start 144.093052 64.93199) (end 153.893534 64.93199) (width 0.4) (layer F.Cu) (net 7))
 (segment (start 143.891 65.134042) (end 144.093052 64.93199) (width 0.4) (layer F.Cu) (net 7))
 (segment (start 143.891 66.802) (end 143.891 65.134042) (width 0.4) (layer F.Cu) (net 7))
 (segment (start 154.686 59.944) (end 154.686 62.330291) (width 0.4) (layer F.Cu) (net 14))
 (segment (start 159.157709 66.802) (end 161.798 66.802) (width 0.4) (layer F.Cu) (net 14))
 (segment (start 154.686 62.330291) (end 159.157709 66.802) (width 0.4) (layer F.Cu) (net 14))
 (segment (start 160.138 73.533) (end 160.274 73.669) (width 0.6) (layer F.Cu) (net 4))
 (segment (start 157.988 73.533) (end 160.138 73.533) (width 0.6) (layer F.Cu) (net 4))
 (segment (start 152.4 58.674) (end 152.146 58.928) (width 0.4) (layer F.Cu) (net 15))
 (segment (start 155.956 59.363998) (end 155.266002 58.674) (width 0.4) (layer F.Cu) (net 15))
 (segment (start 155.266002 58.674) (end 152.4 58.674) (width 0.4) (layer F.Cu) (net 15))
 (segment (start 155.956 62.751749) (end 155.956 59.363998) (width 0.4) (layer F.Cu) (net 15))
 (segment (start 152.146 58.928) (end 152.146 59.944) (width 0.4) (layer F.Cu) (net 15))
 (segment (start 158.75625 65.551999) (end 155.956 62.751749) (width 0.4) (layer F.Cu) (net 15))
 (segment (start 162.398001 65.551999) (end 158.75625 65.551999) (width 0.4) (layer F.Cu) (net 15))
 (segment (start 163.648002 66.802) (end 162.398001 65.551999) (width 0.4) (layer F.Cu) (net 15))
 (segment (start 164.338 66.802) (end 163.648002 66.802) (width 0.4) (layer F.Cu) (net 15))
 (segment (start 160.700989 71.192011) (end 160.274 71.619) (width 0.4) (layer F.Cu) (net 17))
 (segment (start 162.646533 71.192011) (end 160.700989 71.192011) (width 0.4) (layer F.Cu) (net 17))
 (segment (start 164.918002 70.612) (end 163.226544 70.612) (width 0.4) (layer F.Cu) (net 17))
 (segment (start 163.226544 70.612) (end 162.646533 71.192011) (width 0.4) (layer F.Cu) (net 17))
 (segment (start 166.188002 69.342) (end 164.918002 70.612) (width 0.4) (layer F.Cu) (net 17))
 (segment (start 166.878 69.342) (end 166.188002 69.342) (width 0.4) (layer F.Cu) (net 17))
 (segment (start 157.988 76.2) (end 159.766 76.2) (width 0.4) (layer F.Cu) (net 10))
 (segment (start 160.1705 76.6045) (end 160.1705 78.232) (width 0.4) (layer F.Cu) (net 10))
 (segment (start 159.766 76.2) (end 160.1705 76.6045) (width 0.4) (layer F.Cu) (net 10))
 (segment (start 145.288 76.2) (end 147.828 76.2) (width 0.6) (layer F.Cu) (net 1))
 (segment (start 158.3455 78.232) (end 156.6145 78.232) (width 0.4) (layer F.Cu) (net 11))
 (segment (start 156.6145 77.3665) (end 156.6145 78.232) (width 0.4) (layer F.Cu) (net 11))
 (segment (start 155.448 76.2) (end 156.6145 77.3665) (width 0.4) (layer F.Cu) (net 11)))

